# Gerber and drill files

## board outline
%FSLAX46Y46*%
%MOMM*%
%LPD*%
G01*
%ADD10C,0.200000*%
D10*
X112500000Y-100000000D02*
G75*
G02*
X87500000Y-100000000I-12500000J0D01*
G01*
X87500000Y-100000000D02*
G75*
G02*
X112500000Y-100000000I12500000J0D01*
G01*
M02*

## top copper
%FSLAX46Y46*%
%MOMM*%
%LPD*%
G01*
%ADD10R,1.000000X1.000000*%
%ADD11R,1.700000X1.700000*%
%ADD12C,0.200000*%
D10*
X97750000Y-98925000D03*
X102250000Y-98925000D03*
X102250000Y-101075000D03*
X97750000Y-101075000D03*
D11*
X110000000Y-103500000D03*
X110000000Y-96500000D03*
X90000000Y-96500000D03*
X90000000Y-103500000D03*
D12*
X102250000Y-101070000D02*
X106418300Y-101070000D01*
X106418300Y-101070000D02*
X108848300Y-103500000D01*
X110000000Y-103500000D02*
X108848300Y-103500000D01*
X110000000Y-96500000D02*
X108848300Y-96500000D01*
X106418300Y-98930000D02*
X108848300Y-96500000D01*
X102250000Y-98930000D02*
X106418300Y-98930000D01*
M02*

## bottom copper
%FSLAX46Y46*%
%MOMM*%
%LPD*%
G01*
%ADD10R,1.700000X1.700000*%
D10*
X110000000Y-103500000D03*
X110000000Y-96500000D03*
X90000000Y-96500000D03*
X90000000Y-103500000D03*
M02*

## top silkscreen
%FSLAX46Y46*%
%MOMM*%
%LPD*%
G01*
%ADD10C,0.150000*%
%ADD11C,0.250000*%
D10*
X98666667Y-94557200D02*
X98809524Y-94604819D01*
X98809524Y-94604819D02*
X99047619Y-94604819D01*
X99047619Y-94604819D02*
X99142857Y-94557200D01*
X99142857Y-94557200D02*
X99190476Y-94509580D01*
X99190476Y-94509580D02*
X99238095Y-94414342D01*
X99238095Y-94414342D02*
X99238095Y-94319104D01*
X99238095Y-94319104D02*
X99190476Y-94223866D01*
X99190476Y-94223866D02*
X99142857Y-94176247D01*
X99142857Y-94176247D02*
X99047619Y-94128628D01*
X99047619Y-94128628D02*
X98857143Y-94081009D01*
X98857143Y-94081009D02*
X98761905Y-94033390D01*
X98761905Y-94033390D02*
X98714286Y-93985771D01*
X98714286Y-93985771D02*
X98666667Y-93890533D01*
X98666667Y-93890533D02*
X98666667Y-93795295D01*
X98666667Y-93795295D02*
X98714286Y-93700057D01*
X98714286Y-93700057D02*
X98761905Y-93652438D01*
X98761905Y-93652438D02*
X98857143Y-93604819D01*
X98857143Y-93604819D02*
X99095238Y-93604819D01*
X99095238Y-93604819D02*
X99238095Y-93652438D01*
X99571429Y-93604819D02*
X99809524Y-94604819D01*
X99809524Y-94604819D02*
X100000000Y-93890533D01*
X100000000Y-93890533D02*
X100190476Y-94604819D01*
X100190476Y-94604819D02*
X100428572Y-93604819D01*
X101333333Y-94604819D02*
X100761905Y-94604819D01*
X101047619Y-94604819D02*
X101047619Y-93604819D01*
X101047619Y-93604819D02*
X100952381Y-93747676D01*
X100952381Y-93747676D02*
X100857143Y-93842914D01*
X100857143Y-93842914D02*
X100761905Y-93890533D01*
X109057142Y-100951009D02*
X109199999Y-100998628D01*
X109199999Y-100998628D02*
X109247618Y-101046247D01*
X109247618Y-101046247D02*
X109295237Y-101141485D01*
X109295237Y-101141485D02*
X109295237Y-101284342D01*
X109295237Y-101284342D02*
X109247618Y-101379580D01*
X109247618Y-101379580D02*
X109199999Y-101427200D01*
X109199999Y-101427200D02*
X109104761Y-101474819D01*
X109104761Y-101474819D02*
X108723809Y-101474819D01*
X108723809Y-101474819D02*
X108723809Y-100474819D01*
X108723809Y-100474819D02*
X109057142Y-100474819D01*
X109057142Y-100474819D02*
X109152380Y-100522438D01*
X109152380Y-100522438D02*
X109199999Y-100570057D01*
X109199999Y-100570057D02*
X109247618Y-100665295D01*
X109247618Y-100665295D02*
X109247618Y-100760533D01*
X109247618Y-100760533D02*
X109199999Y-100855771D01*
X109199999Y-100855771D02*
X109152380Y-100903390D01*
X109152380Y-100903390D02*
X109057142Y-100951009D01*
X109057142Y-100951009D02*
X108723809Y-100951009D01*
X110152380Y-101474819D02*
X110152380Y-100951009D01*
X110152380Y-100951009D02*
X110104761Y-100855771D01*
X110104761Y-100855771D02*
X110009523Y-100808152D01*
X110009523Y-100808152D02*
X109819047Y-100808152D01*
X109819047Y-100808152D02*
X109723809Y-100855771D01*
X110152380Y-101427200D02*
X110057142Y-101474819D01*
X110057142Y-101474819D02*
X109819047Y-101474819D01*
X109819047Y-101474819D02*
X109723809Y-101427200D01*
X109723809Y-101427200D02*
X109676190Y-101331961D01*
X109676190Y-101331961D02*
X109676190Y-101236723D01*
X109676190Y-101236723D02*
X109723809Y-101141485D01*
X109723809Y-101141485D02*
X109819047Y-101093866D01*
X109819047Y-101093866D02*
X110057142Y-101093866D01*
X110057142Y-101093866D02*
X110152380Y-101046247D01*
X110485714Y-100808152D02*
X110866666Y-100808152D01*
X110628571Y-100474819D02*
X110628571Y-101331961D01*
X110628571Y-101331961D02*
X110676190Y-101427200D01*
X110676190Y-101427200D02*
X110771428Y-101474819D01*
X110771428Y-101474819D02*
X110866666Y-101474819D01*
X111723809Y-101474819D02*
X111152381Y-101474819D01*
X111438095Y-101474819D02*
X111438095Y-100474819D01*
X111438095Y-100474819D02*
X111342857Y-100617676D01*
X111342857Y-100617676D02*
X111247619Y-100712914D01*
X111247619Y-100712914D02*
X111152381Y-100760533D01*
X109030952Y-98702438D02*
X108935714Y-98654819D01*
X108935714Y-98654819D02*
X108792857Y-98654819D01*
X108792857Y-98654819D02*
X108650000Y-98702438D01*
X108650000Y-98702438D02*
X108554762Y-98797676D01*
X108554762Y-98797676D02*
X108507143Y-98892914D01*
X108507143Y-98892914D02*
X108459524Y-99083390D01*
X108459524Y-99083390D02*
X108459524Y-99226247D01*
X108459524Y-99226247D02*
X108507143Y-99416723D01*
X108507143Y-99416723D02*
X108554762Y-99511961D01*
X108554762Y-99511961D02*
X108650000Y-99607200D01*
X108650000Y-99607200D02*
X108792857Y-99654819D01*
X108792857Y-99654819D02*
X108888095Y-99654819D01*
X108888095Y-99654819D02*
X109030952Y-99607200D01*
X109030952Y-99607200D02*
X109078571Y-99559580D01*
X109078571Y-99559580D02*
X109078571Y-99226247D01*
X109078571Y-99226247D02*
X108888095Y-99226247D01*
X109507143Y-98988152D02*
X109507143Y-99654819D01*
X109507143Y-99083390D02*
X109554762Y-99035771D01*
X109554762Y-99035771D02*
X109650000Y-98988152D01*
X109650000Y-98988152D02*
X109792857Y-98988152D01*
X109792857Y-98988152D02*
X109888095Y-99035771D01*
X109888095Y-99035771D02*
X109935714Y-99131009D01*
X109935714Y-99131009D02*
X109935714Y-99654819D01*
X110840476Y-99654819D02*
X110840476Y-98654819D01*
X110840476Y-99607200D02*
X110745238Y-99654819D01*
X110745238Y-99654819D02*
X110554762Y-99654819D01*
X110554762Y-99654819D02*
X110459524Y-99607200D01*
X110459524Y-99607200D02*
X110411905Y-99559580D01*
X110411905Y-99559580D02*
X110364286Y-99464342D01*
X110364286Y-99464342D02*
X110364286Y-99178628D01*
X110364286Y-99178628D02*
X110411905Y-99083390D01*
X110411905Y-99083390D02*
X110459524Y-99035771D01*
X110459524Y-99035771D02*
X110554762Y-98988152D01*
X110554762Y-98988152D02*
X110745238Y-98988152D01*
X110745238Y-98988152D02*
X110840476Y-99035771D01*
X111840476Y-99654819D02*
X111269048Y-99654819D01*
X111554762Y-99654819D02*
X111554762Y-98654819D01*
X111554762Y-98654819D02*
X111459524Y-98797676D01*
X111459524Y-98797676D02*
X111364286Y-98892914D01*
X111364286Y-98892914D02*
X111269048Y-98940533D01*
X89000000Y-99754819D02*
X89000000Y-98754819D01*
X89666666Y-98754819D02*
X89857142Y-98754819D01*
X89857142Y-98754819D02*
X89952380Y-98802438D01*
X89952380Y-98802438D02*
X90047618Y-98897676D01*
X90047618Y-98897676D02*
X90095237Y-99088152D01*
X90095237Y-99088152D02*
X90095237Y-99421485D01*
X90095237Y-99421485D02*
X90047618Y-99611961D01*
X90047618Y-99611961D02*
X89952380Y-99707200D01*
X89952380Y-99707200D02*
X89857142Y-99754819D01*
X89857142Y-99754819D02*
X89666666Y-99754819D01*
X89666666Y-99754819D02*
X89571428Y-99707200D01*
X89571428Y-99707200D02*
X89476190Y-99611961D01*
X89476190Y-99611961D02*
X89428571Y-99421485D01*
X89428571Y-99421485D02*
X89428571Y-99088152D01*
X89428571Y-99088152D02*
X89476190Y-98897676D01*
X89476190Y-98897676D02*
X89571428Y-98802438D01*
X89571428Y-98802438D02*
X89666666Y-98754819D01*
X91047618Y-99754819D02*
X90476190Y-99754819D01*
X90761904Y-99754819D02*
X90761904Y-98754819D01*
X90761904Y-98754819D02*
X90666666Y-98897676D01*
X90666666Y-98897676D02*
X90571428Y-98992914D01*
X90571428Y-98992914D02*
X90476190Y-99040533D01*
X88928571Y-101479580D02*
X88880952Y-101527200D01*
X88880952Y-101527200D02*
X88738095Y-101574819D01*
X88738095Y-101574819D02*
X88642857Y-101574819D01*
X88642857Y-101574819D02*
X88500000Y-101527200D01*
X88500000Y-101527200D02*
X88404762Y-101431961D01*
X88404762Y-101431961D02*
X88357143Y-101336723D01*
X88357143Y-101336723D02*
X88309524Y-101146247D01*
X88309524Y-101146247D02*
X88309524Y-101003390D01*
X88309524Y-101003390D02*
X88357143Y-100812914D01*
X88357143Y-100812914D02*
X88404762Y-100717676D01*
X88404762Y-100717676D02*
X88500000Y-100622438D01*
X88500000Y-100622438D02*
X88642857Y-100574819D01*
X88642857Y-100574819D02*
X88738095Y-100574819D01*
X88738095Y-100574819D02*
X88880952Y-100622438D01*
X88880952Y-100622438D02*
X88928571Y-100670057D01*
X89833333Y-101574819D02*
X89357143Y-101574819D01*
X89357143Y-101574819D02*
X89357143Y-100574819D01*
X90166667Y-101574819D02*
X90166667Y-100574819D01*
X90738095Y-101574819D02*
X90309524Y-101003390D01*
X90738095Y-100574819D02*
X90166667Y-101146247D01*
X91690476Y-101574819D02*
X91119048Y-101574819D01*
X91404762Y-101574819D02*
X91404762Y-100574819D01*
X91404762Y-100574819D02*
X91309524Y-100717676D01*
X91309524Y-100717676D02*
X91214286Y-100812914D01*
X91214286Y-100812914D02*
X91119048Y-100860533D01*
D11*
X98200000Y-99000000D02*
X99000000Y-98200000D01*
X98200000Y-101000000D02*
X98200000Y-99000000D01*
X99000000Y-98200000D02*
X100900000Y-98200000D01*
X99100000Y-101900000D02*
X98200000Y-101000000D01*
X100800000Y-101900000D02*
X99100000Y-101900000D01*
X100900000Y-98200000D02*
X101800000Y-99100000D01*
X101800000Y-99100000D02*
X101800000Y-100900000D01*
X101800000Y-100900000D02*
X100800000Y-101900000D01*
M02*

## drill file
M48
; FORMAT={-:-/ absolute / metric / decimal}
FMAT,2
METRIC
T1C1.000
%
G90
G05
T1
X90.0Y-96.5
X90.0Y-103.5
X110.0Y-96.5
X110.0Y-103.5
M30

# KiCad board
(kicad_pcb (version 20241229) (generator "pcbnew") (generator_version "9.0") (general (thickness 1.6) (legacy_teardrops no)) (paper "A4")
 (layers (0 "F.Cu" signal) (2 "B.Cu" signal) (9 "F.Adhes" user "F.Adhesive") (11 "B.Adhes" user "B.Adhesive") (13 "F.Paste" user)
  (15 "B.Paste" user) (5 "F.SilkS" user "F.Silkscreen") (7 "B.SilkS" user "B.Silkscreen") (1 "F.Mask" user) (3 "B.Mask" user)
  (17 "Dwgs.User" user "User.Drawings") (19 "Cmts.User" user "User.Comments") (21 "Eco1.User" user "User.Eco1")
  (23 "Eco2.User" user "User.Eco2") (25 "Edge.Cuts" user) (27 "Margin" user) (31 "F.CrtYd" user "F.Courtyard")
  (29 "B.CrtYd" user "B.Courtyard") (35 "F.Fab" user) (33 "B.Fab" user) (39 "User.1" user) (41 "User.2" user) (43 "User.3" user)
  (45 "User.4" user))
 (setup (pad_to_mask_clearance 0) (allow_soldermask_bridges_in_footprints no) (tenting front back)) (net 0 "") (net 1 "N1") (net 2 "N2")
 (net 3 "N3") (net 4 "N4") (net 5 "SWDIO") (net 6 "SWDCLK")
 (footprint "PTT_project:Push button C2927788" (layer "F.Cu") (at 100 100)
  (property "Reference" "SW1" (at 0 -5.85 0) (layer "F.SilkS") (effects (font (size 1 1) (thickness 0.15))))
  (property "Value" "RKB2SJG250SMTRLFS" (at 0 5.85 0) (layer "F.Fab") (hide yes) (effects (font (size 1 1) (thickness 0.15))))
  (fp_line (start -1.8 -1) (end -1 -1.8) (stroke (width 0.25) (type solid)) (layer "F.SilkS"))
  (fp_line (start -1.8 1) (end -1.8 -1) (stroke (width 0.25) (type solid)) (layer "F.SilkS"))
  (fp_line (start -1 -1.8) (end 0.9 -1.8) (stroke (width 0.25) (type solid)) (layer "F.SilkS"))
  (fp_line (start -0.9 1.9) (end -1.8 1) (stroke (width 0.25) (type solid)) (layer "F.SilkS"))
  (fp_line (start 0.8 1.9) (end -0.9 1.9) (stroke (width 0.25) (type solid)) (layer "F.SilkS"))
  (fp_line (start 0.9 -1.8) (end 1.8 -0.9) (stroke (width 0.25) (type solid)) (layer "F.SilkS"))
  (fp_line (start 1.8 -0.9) (end 1.8 0.9) (stroke (width 0.25) (type solid)) (layer "F.SilkS"))
  (fp_line (start 1.8 0.9) (end 0.8 1.9) (stroke (width 0.25) (type solid)) (layer "F.SilkS"))
  (pad "1" smd rect (at -2.25 -1.075) (size 1 1) (layers "F.Cu" "F.Mask" "F.Paste") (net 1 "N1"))
  (pad "2" smd rect (at 2.25 -1.075) (size 1 1) (layers "F.Cu" "F.Mask" "F.Paste") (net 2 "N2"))
  (pad "3" smd rect (at 2.25 1.075) (size 1 1) (layers "F.Cu" "F.Mask" "F.Paste") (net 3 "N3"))
  (pad "4" smd rect (at -2.25 1.075) (size 1 1) (layers "F.Cu" "F.Mask" "F.Paste") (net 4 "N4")))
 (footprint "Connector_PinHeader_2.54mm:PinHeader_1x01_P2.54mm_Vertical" (layer "B.Cu") (at 110 103.5 180)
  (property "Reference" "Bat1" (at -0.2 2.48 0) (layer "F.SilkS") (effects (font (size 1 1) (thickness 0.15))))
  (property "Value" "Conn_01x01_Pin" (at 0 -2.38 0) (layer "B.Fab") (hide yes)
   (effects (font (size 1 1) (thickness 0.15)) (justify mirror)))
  (pad "1" thru_hole rect (at 0 0 180) (size 1.7 1.7) (drill 1) (layers "*.Cu" "*.Mask") (remove_unused_layers no) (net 4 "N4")))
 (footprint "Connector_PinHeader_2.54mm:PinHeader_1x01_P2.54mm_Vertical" (layer "B.Cu") (at 110 96.5 180)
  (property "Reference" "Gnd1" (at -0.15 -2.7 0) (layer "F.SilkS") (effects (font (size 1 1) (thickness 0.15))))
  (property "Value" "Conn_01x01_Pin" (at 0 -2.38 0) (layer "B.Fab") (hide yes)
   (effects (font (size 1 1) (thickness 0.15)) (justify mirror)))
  (pad "1" thru_hole rect (at 0 0 180) (size 1.7 1.7) (drill 1) (layers "*.Cu" "*.Mask") (remove_unused_layers no) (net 2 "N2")))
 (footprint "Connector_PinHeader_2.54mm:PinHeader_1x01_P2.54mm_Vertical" (layer "B.Cu") (at 90 96.5 180)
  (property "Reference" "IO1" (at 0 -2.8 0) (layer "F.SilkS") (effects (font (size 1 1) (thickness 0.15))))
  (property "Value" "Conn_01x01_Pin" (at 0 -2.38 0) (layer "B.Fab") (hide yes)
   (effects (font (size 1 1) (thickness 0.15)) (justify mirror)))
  (pad "1" thru_hole rect (at 0 0 180) (size 1.7 1.7) (drill 1) (layers "*.Cu" "*.Mask") (remove_unused_layers no) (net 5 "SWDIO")))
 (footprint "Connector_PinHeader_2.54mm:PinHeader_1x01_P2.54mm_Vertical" (layer "B.Cu") (at 90 103.5 180)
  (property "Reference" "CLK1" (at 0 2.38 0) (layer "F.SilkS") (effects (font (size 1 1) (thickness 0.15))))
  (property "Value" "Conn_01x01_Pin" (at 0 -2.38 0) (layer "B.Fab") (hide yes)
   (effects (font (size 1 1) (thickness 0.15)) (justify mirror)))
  (pad "1" thru_hole rect (at 0 0 180) (size 1.7 1.7) (drill 1) (layers "*.Cu" "*.Mask") (remove_unused_layers no) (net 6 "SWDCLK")))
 (gr_circle (center 100 100) (end 112.5 100) (stroke (width 0.2) (type solid)) (fill no) (layer "Edge.Cuts"))
 (segment (start 102.25 101.07) (end 106.4183 101.07) (width 0.2) (layer "F.Cu") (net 4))
 (segment (start 106.4183 101.07) (end 108.8483 103.5) (width 0.2) (layer "F.Cu") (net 4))
 (segment (start 110 103.5) (end 108.8483 103.5) (width 0.2) (layer "F.Cu") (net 4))
 (segment (start 110 96.5) (end 108.8483 96.5) (width 0.2) (layer "F.Cu") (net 2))
 (segment (start 106.4183 98.93) (end 108.8483 96.5) (width 0.2) (layer "F.Cu") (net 2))
 (segment (start 102.25 98.93) (end 106.4183 98.93) (width 0.2) (layer "F.Cu") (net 2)))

